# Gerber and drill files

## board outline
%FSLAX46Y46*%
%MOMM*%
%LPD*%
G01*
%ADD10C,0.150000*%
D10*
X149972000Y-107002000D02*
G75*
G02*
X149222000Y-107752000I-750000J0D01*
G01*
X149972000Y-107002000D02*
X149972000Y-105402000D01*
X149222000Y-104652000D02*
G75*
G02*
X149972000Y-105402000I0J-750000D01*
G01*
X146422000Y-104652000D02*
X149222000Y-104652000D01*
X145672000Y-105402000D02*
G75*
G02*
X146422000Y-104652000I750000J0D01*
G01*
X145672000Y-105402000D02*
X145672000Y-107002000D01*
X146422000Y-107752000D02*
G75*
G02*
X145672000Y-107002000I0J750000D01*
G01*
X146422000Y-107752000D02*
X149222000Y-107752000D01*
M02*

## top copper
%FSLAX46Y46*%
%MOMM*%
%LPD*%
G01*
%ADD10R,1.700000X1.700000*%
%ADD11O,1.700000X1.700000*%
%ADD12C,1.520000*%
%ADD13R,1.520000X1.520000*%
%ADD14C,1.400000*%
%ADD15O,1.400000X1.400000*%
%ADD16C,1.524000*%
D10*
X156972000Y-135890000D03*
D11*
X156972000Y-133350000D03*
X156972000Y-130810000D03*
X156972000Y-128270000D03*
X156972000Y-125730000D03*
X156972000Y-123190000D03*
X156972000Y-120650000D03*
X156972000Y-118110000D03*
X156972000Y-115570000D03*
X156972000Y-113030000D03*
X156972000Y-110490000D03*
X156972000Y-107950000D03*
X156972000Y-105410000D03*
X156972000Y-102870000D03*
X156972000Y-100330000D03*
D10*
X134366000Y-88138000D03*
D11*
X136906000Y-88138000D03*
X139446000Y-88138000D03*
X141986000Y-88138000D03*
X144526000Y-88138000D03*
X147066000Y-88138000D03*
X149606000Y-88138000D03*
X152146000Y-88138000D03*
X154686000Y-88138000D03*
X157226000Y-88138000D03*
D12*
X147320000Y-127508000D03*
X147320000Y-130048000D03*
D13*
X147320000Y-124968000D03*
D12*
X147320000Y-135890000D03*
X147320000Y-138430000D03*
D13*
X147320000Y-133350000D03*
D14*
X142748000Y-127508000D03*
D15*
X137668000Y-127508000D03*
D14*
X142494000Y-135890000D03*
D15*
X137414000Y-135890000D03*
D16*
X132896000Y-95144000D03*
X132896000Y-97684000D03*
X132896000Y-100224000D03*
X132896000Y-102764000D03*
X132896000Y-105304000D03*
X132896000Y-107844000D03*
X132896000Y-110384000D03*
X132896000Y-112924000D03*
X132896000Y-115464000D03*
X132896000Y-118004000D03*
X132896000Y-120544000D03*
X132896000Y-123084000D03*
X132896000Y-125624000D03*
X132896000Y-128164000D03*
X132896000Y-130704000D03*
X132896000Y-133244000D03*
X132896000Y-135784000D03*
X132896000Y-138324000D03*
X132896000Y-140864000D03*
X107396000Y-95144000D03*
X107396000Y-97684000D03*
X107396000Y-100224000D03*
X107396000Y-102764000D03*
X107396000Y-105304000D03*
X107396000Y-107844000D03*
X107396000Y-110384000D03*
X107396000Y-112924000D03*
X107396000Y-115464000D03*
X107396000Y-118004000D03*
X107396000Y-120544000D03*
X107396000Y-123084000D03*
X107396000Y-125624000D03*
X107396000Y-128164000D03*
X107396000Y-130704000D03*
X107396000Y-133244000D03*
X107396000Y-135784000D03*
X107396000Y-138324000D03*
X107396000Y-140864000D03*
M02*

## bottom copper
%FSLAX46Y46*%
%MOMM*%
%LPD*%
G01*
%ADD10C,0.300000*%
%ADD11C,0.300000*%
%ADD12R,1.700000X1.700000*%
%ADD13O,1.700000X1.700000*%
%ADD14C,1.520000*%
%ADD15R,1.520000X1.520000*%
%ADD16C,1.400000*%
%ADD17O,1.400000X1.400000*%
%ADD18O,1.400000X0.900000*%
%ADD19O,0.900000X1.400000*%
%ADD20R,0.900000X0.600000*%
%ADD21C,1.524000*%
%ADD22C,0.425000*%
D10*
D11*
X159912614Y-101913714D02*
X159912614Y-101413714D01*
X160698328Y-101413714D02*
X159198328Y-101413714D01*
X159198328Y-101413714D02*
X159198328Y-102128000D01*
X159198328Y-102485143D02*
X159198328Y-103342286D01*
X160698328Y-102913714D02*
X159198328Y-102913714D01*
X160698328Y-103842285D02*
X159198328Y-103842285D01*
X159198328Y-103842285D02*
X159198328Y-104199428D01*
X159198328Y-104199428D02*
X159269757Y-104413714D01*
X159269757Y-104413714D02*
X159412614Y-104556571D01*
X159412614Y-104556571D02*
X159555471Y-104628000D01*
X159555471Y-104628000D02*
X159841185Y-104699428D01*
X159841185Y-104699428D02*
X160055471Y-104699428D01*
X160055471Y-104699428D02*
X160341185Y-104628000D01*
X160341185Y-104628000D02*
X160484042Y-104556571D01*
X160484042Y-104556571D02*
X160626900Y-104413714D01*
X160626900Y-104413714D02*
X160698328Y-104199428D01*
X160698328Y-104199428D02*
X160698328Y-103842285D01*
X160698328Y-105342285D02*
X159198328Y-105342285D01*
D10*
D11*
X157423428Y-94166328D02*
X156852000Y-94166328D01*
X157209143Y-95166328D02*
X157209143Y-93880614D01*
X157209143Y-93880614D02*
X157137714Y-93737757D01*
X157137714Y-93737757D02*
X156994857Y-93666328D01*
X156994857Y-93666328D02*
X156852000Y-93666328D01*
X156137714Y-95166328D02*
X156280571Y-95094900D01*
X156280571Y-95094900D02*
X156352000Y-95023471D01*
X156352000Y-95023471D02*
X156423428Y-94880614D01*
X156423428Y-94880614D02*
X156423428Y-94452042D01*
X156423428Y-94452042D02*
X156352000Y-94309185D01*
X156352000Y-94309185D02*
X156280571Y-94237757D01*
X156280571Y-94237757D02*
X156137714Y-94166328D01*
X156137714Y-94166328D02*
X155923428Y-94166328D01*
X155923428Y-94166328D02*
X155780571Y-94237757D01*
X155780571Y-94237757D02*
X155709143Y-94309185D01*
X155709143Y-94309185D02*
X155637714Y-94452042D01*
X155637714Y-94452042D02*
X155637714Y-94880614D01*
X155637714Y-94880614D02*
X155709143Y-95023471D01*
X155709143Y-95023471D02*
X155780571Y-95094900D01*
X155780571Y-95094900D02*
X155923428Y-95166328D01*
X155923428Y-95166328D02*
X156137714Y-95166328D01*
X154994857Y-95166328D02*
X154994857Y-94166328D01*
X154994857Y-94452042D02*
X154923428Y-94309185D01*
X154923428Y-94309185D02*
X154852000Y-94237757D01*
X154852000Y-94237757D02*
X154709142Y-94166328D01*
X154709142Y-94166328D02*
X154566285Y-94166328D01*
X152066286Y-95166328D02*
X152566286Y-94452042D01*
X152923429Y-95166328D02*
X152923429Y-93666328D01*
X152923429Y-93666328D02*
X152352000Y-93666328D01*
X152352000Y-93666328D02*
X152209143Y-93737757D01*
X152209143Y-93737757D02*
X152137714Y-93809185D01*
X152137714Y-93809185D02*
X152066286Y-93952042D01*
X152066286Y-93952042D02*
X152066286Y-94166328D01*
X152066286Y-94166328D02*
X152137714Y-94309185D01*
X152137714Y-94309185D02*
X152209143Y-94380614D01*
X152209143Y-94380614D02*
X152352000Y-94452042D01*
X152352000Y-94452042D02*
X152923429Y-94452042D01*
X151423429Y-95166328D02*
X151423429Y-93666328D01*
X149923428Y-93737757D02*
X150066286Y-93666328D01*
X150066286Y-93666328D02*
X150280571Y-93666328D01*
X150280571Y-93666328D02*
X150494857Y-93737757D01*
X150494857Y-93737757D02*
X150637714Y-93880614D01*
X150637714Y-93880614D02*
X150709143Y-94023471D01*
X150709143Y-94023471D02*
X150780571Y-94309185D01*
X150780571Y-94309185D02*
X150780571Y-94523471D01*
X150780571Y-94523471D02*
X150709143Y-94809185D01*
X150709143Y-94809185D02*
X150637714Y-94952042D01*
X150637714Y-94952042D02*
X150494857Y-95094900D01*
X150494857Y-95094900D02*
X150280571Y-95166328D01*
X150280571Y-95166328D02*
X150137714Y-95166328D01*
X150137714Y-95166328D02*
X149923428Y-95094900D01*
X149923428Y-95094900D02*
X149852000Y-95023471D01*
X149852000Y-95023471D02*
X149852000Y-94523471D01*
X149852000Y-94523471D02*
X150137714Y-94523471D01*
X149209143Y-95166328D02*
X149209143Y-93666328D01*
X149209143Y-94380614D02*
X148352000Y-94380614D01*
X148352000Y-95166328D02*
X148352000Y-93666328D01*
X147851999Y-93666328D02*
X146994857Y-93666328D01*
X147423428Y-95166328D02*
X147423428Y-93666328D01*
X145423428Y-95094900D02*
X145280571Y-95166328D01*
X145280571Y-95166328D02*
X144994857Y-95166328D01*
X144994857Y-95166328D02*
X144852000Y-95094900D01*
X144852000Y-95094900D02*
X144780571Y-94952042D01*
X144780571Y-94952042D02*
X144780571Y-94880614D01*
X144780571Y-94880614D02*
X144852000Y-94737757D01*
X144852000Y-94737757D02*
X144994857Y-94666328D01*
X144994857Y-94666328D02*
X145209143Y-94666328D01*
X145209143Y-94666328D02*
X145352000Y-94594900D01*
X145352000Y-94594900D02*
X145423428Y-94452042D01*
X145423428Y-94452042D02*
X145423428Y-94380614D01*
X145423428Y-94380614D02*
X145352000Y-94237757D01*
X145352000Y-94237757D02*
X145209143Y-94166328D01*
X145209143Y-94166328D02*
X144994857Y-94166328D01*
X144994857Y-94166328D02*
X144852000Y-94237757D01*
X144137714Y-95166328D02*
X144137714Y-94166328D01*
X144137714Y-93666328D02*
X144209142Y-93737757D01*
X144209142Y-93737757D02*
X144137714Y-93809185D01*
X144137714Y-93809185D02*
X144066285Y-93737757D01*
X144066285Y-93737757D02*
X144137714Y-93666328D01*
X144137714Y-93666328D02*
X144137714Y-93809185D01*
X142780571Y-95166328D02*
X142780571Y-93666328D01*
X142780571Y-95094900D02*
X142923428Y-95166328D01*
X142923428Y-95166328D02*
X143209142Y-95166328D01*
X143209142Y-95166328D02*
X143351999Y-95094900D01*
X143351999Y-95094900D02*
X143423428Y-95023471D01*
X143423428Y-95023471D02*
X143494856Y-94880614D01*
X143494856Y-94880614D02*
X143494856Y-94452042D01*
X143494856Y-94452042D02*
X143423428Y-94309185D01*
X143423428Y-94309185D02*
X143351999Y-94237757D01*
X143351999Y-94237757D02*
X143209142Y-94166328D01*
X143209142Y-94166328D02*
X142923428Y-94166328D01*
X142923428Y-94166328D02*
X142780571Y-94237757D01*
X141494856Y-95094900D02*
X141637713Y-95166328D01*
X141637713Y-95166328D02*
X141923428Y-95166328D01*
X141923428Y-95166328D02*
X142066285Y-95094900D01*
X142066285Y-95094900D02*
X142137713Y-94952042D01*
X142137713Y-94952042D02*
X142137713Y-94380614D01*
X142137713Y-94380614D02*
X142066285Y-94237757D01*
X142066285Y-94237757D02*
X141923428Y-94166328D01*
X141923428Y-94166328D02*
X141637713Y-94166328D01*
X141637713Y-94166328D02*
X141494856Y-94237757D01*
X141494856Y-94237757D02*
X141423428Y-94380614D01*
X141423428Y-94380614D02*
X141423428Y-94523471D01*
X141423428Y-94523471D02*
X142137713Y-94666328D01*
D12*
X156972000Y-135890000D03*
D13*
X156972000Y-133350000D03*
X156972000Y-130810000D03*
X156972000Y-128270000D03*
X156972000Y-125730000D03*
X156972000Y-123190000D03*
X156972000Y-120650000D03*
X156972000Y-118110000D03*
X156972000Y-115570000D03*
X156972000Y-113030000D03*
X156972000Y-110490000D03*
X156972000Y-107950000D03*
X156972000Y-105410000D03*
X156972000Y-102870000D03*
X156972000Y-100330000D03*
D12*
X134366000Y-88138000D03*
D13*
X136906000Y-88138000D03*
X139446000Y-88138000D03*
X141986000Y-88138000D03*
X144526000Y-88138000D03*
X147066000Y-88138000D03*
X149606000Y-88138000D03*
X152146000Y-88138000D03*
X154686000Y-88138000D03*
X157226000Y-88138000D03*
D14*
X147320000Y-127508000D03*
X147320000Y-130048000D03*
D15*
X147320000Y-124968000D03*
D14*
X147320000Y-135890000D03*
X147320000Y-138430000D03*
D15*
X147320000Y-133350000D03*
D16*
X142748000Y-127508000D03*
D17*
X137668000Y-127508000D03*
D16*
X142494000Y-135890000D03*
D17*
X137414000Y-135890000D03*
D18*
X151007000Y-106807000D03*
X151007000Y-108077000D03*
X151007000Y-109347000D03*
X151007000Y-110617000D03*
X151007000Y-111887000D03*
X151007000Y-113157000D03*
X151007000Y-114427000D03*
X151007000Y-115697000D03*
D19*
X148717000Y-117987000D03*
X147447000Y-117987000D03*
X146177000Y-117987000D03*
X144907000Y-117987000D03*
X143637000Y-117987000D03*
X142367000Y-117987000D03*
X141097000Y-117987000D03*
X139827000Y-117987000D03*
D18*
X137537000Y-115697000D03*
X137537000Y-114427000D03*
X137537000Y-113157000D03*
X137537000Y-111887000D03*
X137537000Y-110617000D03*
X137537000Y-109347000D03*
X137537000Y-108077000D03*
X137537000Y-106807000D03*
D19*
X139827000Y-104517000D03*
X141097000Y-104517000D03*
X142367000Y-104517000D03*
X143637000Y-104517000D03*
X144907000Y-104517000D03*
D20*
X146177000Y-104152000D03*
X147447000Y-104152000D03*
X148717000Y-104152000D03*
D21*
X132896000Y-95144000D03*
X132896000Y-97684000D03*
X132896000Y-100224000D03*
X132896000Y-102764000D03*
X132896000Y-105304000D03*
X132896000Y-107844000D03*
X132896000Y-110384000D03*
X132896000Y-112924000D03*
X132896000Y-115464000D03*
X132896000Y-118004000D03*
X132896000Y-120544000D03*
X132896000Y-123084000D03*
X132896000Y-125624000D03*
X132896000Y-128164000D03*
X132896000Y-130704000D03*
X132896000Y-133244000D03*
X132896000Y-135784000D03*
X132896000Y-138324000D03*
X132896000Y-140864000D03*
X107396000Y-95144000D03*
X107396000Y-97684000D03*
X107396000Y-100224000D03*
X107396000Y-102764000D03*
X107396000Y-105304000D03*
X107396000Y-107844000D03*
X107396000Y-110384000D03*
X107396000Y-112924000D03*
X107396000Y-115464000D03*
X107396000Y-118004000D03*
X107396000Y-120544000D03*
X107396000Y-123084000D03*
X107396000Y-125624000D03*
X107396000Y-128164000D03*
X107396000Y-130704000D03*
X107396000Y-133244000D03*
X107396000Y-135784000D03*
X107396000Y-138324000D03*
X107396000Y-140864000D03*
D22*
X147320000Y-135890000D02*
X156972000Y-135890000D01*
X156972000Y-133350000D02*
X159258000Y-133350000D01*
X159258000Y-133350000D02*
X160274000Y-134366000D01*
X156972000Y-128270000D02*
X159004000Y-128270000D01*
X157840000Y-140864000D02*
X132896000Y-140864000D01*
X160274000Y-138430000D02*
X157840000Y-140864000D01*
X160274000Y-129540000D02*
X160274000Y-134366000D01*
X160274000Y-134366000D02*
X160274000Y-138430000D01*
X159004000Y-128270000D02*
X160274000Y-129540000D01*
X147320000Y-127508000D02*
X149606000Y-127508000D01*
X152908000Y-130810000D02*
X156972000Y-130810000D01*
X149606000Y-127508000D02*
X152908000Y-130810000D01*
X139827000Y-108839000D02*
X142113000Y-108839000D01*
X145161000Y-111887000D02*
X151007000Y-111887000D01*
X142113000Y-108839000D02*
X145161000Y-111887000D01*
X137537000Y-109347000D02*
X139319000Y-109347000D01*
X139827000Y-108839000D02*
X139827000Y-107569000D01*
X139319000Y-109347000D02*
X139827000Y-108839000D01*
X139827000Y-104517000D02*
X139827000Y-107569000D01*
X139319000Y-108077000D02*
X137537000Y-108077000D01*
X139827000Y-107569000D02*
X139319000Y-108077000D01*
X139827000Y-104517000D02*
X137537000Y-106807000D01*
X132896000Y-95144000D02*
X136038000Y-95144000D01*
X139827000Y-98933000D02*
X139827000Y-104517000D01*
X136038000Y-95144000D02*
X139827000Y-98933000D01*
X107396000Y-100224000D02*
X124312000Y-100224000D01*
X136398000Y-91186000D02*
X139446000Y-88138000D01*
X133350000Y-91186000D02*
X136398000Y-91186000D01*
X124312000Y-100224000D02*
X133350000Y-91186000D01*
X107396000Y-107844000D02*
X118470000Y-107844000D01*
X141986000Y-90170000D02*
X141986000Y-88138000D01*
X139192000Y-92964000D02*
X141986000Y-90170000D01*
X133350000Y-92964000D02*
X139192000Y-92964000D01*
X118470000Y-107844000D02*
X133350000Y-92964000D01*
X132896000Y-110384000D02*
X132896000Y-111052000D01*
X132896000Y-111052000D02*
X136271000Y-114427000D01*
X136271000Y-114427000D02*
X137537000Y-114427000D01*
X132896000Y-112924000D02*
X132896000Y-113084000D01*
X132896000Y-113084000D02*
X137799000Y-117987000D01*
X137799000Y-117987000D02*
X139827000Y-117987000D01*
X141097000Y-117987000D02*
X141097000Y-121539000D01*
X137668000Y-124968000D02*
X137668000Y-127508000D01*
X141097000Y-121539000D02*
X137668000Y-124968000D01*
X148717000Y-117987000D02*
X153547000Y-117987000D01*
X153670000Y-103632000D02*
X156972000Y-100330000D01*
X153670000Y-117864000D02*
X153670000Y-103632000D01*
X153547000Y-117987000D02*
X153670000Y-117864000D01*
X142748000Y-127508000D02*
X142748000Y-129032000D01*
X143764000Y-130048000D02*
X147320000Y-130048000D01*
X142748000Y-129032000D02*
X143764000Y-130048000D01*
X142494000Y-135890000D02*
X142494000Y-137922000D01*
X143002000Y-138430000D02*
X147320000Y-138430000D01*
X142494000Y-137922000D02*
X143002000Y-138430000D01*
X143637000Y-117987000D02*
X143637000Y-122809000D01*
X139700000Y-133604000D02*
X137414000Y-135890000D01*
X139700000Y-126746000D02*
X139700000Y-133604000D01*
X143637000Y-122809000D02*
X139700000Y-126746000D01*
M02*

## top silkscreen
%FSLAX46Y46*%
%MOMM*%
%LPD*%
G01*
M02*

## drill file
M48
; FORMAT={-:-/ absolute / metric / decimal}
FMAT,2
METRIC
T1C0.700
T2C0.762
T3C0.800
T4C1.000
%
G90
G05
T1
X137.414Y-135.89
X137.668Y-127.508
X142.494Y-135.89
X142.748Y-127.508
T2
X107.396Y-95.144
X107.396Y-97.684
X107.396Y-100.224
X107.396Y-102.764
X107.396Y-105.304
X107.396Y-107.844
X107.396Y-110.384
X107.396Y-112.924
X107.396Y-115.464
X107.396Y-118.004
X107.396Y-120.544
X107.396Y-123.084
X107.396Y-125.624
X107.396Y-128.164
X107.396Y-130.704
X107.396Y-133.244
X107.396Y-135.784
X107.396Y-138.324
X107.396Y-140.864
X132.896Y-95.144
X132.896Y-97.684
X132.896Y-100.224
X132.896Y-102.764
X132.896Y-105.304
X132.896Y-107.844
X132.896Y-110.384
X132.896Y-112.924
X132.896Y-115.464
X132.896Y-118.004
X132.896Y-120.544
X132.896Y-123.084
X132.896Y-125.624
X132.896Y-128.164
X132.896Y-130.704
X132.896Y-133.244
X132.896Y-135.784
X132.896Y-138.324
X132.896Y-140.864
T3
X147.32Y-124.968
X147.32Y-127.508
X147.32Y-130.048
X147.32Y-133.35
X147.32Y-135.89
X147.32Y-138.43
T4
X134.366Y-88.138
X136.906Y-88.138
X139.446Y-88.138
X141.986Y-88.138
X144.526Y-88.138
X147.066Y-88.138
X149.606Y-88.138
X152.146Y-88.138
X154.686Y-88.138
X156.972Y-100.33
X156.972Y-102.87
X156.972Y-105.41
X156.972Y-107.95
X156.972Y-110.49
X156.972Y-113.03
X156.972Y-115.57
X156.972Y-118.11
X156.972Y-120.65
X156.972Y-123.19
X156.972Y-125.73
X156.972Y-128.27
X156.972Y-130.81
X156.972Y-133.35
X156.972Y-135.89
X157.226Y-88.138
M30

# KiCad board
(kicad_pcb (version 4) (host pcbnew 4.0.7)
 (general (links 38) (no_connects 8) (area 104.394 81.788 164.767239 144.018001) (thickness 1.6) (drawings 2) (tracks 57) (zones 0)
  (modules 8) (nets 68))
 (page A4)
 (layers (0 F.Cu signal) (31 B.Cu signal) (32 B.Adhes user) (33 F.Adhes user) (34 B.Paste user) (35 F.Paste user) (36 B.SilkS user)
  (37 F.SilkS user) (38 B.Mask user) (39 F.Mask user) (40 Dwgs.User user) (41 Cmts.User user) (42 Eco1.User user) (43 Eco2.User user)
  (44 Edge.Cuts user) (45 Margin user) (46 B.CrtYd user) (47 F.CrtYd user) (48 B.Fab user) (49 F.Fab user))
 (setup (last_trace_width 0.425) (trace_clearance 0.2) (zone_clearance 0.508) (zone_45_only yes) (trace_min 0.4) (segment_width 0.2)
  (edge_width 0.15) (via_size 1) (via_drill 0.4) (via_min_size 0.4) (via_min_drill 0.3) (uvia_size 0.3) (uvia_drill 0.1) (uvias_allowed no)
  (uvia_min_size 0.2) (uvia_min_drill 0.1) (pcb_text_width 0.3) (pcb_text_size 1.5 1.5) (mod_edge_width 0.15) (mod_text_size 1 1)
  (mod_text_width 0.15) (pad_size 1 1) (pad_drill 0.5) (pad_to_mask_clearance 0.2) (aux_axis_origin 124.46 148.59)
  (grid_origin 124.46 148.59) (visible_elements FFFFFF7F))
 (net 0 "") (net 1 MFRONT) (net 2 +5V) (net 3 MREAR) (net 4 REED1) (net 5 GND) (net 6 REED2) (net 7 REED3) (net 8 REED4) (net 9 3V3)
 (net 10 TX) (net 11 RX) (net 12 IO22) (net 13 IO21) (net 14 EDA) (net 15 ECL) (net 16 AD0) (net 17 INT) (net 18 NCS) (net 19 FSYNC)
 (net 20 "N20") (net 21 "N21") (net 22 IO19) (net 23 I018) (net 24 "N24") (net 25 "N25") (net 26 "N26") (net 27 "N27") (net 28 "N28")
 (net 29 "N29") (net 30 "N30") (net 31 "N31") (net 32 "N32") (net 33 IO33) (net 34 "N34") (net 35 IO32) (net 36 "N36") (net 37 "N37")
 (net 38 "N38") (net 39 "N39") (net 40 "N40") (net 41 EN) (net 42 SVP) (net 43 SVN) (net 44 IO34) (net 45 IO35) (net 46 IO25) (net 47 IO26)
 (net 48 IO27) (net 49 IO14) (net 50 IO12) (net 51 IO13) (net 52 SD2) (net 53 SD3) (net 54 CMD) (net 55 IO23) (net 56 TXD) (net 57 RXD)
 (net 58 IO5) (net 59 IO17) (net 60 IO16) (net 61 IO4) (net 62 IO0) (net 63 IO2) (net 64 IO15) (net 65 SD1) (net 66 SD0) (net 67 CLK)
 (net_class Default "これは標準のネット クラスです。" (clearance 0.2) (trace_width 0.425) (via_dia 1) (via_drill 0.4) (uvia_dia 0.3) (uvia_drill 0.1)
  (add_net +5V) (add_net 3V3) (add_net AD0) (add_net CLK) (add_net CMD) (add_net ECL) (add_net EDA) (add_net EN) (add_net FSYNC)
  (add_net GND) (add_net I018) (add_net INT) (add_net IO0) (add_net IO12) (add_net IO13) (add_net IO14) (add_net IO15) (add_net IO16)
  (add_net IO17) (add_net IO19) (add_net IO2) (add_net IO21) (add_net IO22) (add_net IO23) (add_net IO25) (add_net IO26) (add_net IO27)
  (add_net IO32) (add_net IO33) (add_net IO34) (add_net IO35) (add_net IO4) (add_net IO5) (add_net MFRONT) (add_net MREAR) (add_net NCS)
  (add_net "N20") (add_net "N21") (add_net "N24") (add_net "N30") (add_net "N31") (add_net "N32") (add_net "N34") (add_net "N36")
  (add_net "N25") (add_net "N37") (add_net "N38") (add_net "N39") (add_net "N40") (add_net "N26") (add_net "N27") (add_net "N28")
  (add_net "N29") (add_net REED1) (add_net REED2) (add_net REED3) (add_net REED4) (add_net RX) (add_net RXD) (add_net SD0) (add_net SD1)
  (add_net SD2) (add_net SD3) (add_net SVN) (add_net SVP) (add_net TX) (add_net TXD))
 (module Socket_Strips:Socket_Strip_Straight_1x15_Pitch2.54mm (layer B.Cu) (at 156.972 135.89)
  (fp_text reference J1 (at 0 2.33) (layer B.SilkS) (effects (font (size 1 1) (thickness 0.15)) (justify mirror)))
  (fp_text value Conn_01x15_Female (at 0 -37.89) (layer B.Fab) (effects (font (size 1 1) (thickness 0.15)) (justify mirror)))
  (pad 1 thru_hole rect (at 0 0) (size 1.7 1.7) (drill 1) (layers *.Cu *.Mask) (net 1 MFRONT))
  (pad 2 thru_hole oval (at 0 -2.54) (size 1.7 1.7) (drill 1) (layers *.Cu *.Mask) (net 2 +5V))
  (pad 3 thru_hole oval (at 0 -5.08) (size 1.7 1.7) (drill 1) (layers *.Cu *.Mask) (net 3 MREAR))
  (pad 4 thru_hole oval (at 0 -7.62) (size 1.7 1.7) (drill 1) (layers *.Cu *.Mask) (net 2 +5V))
  (pad 5 thru_hole oval (at 0 -10.16) (size 1.7 1.7) (drill 1) (layers *.Cu *.Mask) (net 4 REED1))
  (pad 6 thru_hole oval (at 0 -12.7) (size 1.7 1.7) (drill 1) (layers *.Cu *.Mask) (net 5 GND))
  (pad 7 thru_hole oval (at 0 -15.24) (size 1.7 1.7) (drill 1) (layers *.Cu *.Mask) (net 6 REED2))
  (pad 8 thru_hole oval (at 0 -17.78) (size 1.7 1.7) (drill 1) (layers *.Cu *.Mask) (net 5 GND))
  (pad 9 thru_hole oval (at 0 -20.32) (size 1.7 1.7) (drill 1) (layers *.Cu *.Mask) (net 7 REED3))
  (pad 10 thru_hole oval (at 0 -22.86) (size 1.7 1.7) (drill 1) (layers *.Cu *.Mask) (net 5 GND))
  (pad 11 thru_hole oval (at 0 -25.4) (size 1.7 1.7) (drill 1) (layers *.Cu *.Mask) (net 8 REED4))
  (pad 12 thru_hole oval (at 0 -27.94) (size 1.7 1.7) (drill 1) (layers *.Cu *.Mask) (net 5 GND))
  (pad 13 thru_hole oval (at 0 -30.48) (size 1.7 1.7) (drill 1) (layers *.Cu *.Mask) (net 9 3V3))
  (pad 14 thru_hole oval (at 0 -33.02) (size 1.7 1.7) (drill 1) (layers *.Cu *.Mask) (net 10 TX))
  (pad 15 thru_hole oval (at 0 -35.56) (size 1.7 1.7) (drill 1) (layers *.Cu *.Mask) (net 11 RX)))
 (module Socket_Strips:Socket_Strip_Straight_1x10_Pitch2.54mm (layer B.Cu) (at 134.366 88.138 270)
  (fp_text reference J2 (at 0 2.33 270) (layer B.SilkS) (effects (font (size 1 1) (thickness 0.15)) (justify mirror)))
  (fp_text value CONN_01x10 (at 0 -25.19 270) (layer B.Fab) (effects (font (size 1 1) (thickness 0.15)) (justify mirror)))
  (pad 1 thru_hole rect (at 0 0 270) (size 1.7 1.7) (drill 1) (layers *.Cu *.Mask) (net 9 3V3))
  (pad 2 thru_hole oval (at 0 -2.54 270) (size 1.7 1.7) (drill 1) (layers *.Cu *.Mask) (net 5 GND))
  (pad 3 thru_hole oval (at 0 -5.08 270) (size 1.7 1.7) (drill 1) (layers *.Cu *.Mask) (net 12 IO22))
  (pad 4 thru_hole oval (at 0 -7.62 270) (size 1.7 1.7) (drill 1) (layers *.Cu *.Mask) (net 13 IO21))
  (pad 5 thru_hole oval (at 0 -10.16 270) (size 1.7 1.7) (drill 1) (layers *.Cu *.Mask) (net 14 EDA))
  (pad 6 thru_hole oval (at 0 -12.7 270) (size 1.7 1.7) (drill 1) (layers *.Cu *.Mask) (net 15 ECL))
  (pad 7 thru_hole oval (at 0 -15.24 270) (size 1.7 1.7) (drill 1) (layers *.Cu *.Mask) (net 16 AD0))
  (pad 8 thru_hole oval (at 0 -17.78 270) (size 1.7 1.7) (drill 1) (layers *.Cu *.Mask) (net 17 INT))
  (pad 9 thru_hole oval (at 0 -20.32 270) (size 1.7 1.7) (drill 1) (layers *.Cu *.Mask) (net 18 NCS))
  (pad 10 thru_hole oval (at 0 -22.86 270) (size 1.7 1.7) (drill 1) (layers *.Cu *.Mask) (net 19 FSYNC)))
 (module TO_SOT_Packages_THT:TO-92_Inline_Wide (layer B.Cu) (at 147.32 124.968 270)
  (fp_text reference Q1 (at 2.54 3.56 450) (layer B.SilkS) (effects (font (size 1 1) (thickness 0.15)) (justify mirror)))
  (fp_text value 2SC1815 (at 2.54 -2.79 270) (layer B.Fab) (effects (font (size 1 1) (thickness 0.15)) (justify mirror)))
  (pad 2 thru_hole circle (at 2.54 0 180) (size 1.52 1.52) (drill 0.8) (layers *.Cu *.Mask) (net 3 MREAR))
  (pad 3 thru_hole circle (at 5.08 0 180) (size 1.52 1.52) (drill 0.8) (layers *.Cu *.Mask) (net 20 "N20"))
  (pad 1 thru_hole rect (at 0 0 180) (size 1.52 1.52) (drill 0.8) (layers *.Cu *.Mask) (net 5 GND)))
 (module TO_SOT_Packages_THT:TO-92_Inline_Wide (layer B.Cu) (at 147.32 133.35 270)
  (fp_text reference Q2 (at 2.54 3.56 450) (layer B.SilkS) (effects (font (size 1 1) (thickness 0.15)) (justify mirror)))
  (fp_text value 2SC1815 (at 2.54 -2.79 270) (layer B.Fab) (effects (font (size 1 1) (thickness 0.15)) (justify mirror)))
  (pad 2 thru_hole circle (at 2.54 0 180) (size 1.52 1.52) (drill 0.8) (layers *.Cu *.Mask) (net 1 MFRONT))
  (pad 3 thru_hole circle (at 5.08 0 180) (size 1.52 1.52) (drill 0.8) (layers *.Cu *.Mask) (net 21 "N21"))
  (pad 1 thru_hole rect (at 0 0 180) (size 1.52 1.52) (drill 0.8) (layers *.Cu *.Mask) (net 5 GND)))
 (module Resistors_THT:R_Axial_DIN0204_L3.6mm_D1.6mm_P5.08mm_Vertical (layer B.Cu) (at 142.748 127.508 180)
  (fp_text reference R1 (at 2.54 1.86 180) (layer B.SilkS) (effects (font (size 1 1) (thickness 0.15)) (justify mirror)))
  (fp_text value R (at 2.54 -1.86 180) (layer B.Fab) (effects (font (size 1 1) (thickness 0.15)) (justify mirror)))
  (pad 1 thru_hole circle (at 0 0 180) (size 1.4 1.4) (drill 0.7) (layers *.Cu *.Mask) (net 20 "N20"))
  (pad 2 thru_hole oval (at 5.08 0 180) (size 1.4 1.4) (drill 0.7) (layers *.Cu *.Mask) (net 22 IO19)))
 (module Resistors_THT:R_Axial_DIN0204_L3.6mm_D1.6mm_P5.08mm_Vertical (layer B.Cu) (at 142.494 135.89 180)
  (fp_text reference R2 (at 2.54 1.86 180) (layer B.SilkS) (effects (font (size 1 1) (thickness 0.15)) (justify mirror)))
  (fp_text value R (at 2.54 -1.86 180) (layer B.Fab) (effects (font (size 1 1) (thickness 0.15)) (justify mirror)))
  (pad 1 thru_hole circle (at 0 0 180) (size 1.4 1.4) (drill 0.7) (layers *.Cu *.Mask) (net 21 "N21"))
  (pad 2 thru_hole oval (at 5.08 0 180) (size 1.4 1.4) (drill 0.7) (layers *.Cu *.Mask) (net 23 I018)))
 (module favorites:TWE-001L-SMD (layer B.Cu) (at 144.272 111.252 180)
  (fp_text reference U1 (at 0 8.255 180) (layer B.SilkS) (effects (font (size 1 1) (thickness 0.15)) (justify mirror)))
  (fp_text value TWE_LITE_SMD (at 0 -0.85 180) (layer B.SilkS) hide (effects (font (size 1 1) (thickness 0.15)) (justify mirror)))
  (fp_arc (start -4.95 4.25) (end -4.95 3.5) (angle -90) (layer Edge.Cuts) (width 0.15))
  (fp_line (start -5.7 4.25) (end -5.7 5.85) (layer Edge.Cuts) (width 0.15))
  (fp_arc (start -4.95 5.85) (end -5.7 5.85) (angle -90) (layer Edge.Cuts) (width 0.15))
  (fp_line (start -2.15 6.6) (end -4.95 6.6) (layer Edge.Cuts) (width 0.15))
  (fp_arc (start -2.15 5.85) (end -2.15 6.6) (angle -90) (layer Edge.Cuts) (width 0.15))
  (fp_line (start -1.4 5.85) (end -1.4 4.25) (layer Edge.Cuts) (width 0.15))
  (fp_arc (start -2.15 4.25) (end -1.4 4.25) (angle -90) (layer Edge.Cuts) (width 0.15))
  (fp_line (start -2.15 3.5) (end -4.95 3.5) (layer Edge.Cuts) (width 0.15))
  (pad 1 smd oval (at -6.735 4.445 90) (size 0.9 1.4) (layers B.Cu B.Paste B.Mask) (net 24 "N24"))
  (pad 2 smd oval (at -6.735 3.175 90) (size 0.9 1.4) (layers B.Cu B.Paste B.Mask) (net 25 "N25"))
  (pad 3 smd oval (at -6.735 1.905 90) (size 0.9 1.4) (layers B.Cu B.Paste B.Mask) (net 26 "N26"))
  (pad 4 smd oval (at -6.735 0.635 90) (size 0.9 1.4) (layers B.Cu B.Paste B.Mask) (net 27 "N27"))
  (pad 5 smd oval (at -6.735 -0.635 90) (size 0.9 1.4) (layers B.Cu B.Paste B.Mask) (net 9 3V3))
  (pad 6 smd oval (at -6.735 -1.905 90) (size 0.9 1.4) (layers B.Cu B.Paste B.Mask) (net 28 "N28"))
  (pad 7 smd oval (at -6.735 -3.175 90) (size 0.9 1.4) (layers B.Cu B.Paste B.Mask) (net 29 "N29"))
  (pad 8 smd oval (at -6.735 -4.445 90) (size 0.9 1.4) (layers B.Cu B.Paste B.Mask) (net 10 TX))
  (pad 9 smd oval (at -4.445 -6.735 180) (size 0.9 1.4) (layers B.Cu B.Paste B.Mask) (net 11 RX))
  (pad 10 smd oval (at -3.175 -6.735 180) (size 0.9 1.4) (layers B.Cu B.Paste B.Mask) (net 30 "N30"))
  (pad 11 smd oval (at -1.905 -6.735 180) (size 0.9 1.4) (layers B.Cu B.Paste B.Mask) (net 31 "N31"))
  (pad 12 smd oval (at -0.635 -6.735 180) (size 0.9 1.4) (layers B.Cu B.Paste B.Mask) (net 5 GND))
  (pad 13 smd oval (at 0.635 -6.735 180) (size 0.9 1.4) (layers B.Cu B.Paste B.Mask) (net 23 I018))
  (pad 14 smd oval (at 1.905 -6.735 180) (size 0.9 1.4) (layers B.Cu B.Paste B.Mask) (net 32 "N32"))
  (pad 15 smd oval (at 3.175 -6.735 180) (size 0.9 1.4) (layers B.Cu B.Paste B.Mask) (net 22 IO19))
  (pad 16 smd oval (at 4.445 -6.735 180) (size 0.9 1.4) (layers B.Cu B.Paste B.Mask) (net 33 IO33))
  (pad 17 smd oval (at 6.735 -4.445 90) (size 0.9 1.4) (layers B.Cu B.Paste B.Mask) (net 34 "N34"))
  (pad 18 smd oval (at 6.735 -3.175 90) (size 0.9 1.4) (layers B.Cu B.Paste B.Mask) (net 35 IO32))
  (pad 19 smd oval (at 6.735 -1.905 90) (size 0.9 1.4) (layers B.Cu B.Paste B.Mask) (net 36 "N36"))
  (pad 20 smd oval (at 6.735 -0.635 90) (size 0.9 1.4) (layers B.Cu B.Paste B.Mask) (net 5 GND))
  (pad 21 smd oval (at 6.735 0.635 90) (size 0.9 1.4) (layers B.Cu B.Paste B.Mask) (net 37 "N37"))
  (pad 22 smd oval (at 6.735 1.905 90) (size 0.9 1.4) (layers B.Cu B.Paste B.Mask) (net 9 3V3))
  (pad 23 smd oval (at 6.735 3.175 90) (size 0.9 1.4) (layers B.Cu B.Paste B.Mask) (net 9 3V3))
  (pad 24 smd oval (at 6.735 4.445 90) (size 0.9 1.4) (layers B.Cu B.Paste B.Mask) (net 9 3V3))
  (pad 25 smd oval (at 4.445 6.735 180) (size 0.9 1.4) (layers B.Cu B.Paste B.Mask) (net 9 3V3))
  (pad 26 smd oval (at 3.175 6.735 180) (size 0.9 1.4) (layers B.Cu B.Paste B.Mask) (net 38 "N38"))
  (pad 27 smd oval (at 1.905 6.735 180) (size 0.9 1.4) (layers B.Cu B.Paste B.Mask) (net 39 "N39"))
  (pad 28 smd oval (at 0.635 6.735 180) (size 0.9 1.4) (layers B.Cu B.Paste B.Mask) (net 5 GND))
  (pad 29 smd oval (at -0.635 6.735 180) (size 0.9 1.4) (layers B.Cu B.Paste B.Mask) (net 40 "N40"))
  (pad 30 smd rect (at -1.905 7.1 180) (size 0.9 0.6) (layers B.Cu B.Paste B.Mask) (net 5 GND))
  (pad 31 smd rect (at -3.175 7.1 180) (size 0.9 0.6) (layers B.Cu B.Paste B.Mask) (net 5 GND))
  (pad 32 smd rect (at -4.445 7.1 180) (size 0.9 0.6) (layers B.Cu B.Paste B.Mask) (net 5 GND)))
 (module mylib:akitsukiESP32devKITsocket (layer B.Cu) (at 120.396 123.444 180)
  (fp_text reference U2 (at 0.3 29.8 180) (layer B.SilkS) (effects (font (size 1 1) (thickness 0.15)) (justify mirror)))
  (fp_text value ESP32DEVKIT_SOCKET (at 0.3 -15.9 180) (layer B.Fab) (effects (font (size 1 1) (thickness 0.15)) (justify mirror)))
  (pad 1 thru_hole circle (at -12.5 28.3 180) (size 1.524 1.524) (drill 0.762) (layers *.Cu *.Mask) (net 9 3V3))
  (pad 2 thru_hole circle (at -12.5 25.76 180) (size 1.524 1.524) (drill 0.762) (layers *.Cu *.Mask) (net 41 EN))
  (pad 3 thru_hole circle (at -12.5 23.22 180) (size 1.524 1.524) (drill 0.762) (layers *.Cu *.Mask) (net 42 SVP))
  (pad 4 thru_hole circle (at -12.5 20.68 180) (size 1.524 1.524) (drill 0.762) (layers *.Cu *.Mask) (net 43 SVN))
  (pad 5 thru_hole circle (at -12.5 18.14 180) (size 1.524 1.524) (drill 0.762) (layers *.Cu *.Mask) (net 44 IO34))
  (pad 6 thru_hole circle (at -12.5 15.6 180) (size 1.524 1.524) (drill 0.762) (layers *.Cu *.Mask) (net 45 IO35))
  (pad 7 thru_hole circle (at -12.5 13.06 180) (size 1.524 1.524) (drill 0.762) (layers *.Cu *.Mask) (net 35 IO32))
  (pad 8 thru_hole circle (at -12.5 10.52 180) (size 1.524 1.524) (drill 0.762) (layers *.Cu *.Mask) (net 33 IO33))
  (pad 9 thru_hole circle (at -12.5 7.98 180) (size 1.524 1.524) (drill 0.762) (layers *.Cu *.Mask) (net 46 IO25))
  (pad 10 thru_hole circle (at -12.5 5.44 180) (size 1.524 1.524) (drill 0.762) (layers *.Cu *.Mask) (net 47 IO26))
  (pad 11 thru_hole circle (at -12.5 2.9 180) (size 1.524 1.524) (drill 0.762) (layers *.Cu *.Mask) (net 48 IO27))
  (pad 12 thru_hole circle (at -12.5 0.36 180) (size 1.524 1.524) (drill 0.762) (layers *.Cu *.Mask) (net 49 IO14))
  (pad 13 thru_hole circle (at -12.5 -2.18 180) (size 1.524 1.524) (drill 0.762) (layers *.Cu *.Mask) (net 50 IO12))
  (pad 14 thru_hole circle (at -12.5 -4.72 180) (size 1.524 1.524) (drill 0.762) (layers *.Cu *.Mask) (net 5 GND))
  (pad 15 thru_hole circle (at -12.5 -7.26 180) (size 1.524 1.524) (drill 0.762) (layers *.Cu *.Mask) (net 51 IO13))
  (pad 16 thru_hole circle (at -12.5 -9.8 180) (size 1.524 1.524) (drill 0.762) (layers *.Cu *.Mask) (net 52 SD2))
  (pad 17 thru_hole circle (at -12.5 -12.34 180) (size 1.524 1.524) (drill 0.762) (layers *.Cu *.Mask) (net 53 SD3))
  (pad 18 thru_hole circle (at -12.5 -14.88 180) (size 1.524 1.524) (drill 0.762) (layers *.Cu *.Mask) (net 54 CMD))
  (pad 19 thru_hole circle (at -12.5 -17.42 180) (size 1.524 1.524) (drill 0.762) (layers *.Cu *.Mask) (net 2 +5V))
  (pad 20 thru_hole circle (at 13 28.3 180) (size 1.524 1.524) (drill 0.762) (layers *.Cu *.Mask) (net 5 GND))
  (pad 21 thru_hole circle (at 13 25.76 180) (size 1.524 1.524) (drill 0.762) (layers *.Cu *.Mask) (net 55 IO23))
  (pad 22 thru_hole circle (at 13 23.22 180) (size 1.524 1.524) (drill 0.762) (layers *.Cu *.Mask) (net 12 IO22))
  (pad 23 thru_hole circle (at 13 20.68 180) (size 1.524 1.524) (drill 0.762) (layers *.Cu *.Mask) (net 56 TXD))
  (pad 24 thru_hole circle (at 13 18.14 180) (size 1.524 1.524) (drill 0.762) (layers *.Cu *.Mask) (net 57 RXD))
  (pad 25 thru_hole circle (at 13 15.6 180) (size 1.524 1.524) (drill 0.762) (layers *.Cu *.Mask) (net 13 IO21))
  (pad 26 thru_hole circle (at 13 13.06 180) (size 1.524 1.524) (drill 0.762) (layers *.Cu *.Mask) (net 5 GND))
  (pad 27 thru_hole circle (at 13 10.52 180) (size 1.524 1.524) (drill 0.762) (layers *.Cu *.Mask) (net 22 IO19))
  (pad 28 thru_hole circle (at 13 7.98 180) (size 1.524 1.524) (drill 0.762) (layers *.Cu *.Mask) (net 23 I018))
  (pad 29 thru_hole circle (at 13 5.44 180) (size 1.524 1.524) (drill 0.762) (layers *.Cu *.Mask) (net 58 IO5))
  (pad 30 thru_hole circle (at 13 2.9 180) (size 1.524 1.524) (drill 0.762) (layers *.Cu *.Mask) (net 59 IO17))
  (pad 31 thru_hole circle (at 13 0.36 180) (size 1.524 1.524) (drill 0.762) (layers *.Cu *.Mask) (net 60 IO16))
  (pad 32 thru_hole circle (at 13 -2.18 180) (size 1.524 1.524) (drill 0.762) (layers *.Cu *.Mask) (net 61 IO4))
  (pad 33 thru_hole circle (at 13 -4.72 180) (size 1.524 1.524) (drill 0.762) (layers *.Cu *.Mask) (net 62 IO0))
  (pad 34 thru_hole circle (at 13 -7.26 180) (size 1.524 1.524) (drill 0.762) (layers *.Cu *.Mask) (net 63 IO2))
  (pad 35 thru_hole circle (at 13 -9.8 180) (size 1.524 1.524) (drill 0.762) (layers *.Cu *.Mask) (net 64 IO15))
  (pad 36 thru_hole circle (at 13 -12.34 180) (size 1.524 1.524) (drill 0.762) (layers *.Cu *.Mask) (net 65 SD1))
  (pad 37 thru_hole circle (at 13 -14.88 180) (size 1.524 1.524) (drill 0.762) (layers *.Cu *.Mask) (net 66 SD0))
  (pad 38 thru_hole circle (at 13 -17.42 180) (size 1.524 1.524) (drill 0.762) (layers *.Cu *.Mask) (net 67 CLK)))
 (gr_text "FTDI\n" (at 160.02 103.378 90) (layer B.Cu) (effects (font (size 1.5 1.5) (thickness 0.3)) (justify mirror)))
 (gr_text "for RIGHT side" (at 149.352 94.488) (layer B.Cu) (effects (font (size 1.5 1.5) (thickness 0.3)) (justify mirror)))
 (segment (start 147.32 135.89) (end 156.972 135.89) (width 0.425) (layer B.Cu) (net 1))
 (segment (start 156.972 133.35) (end 159.258 133.35) (width 0.425) (layer B.Cu) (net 2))
 (segment (start 159.258 133.35) (end 160.274 134.366) (width 0.425) (layer B.Cu) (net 2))
 (segment (start 156.972 128.27) (end 159.004 128.27) (width 0.425) (layer B.Cu) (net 2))
 (segment (start 157.84 140.864) (end 132.896 140.864) (width 0.425) (layer B.Cu) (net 2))
 (segment (start 160.274 138.43) (end 157.84 140.864) (width 0.425) (layer B.Cu) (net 2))
 (segment (start 160.274 129.54) (end 160.274 134.366) (width 0.425) (layer B.Cu) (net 2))
 (segment (start 160.274 134.366) (end 160.274 138.43) (width 0.425) (layer B.Cu) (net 2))
 (segment (start 159.004 128.27) (end 160.274 129.54) (width 0.425) (layer B.Cu) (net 2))
 (segment (start 147.32 127.508) (end 149.606 127.508) (width 0.425) (layer B.Cu) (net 3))
 (segment (start 152.908 130.81) (end 156.972 130.81) (width 0.425) (layer B.Cu) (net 3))
 (segment (start 149.606 127.508) (end 152.908 130.81) (width 0.425) (layer B.Cu) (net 3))
 (segment (start 139.827 108.839) (end 142.113 108.839) (width 0.425) (layer B.Cu) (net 9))
 (segment (start 145.161 111.887) (end 151.007 111.887) (width 0.425) (layer B.Cu) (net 9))
 (segment (start 142.113 108.839) (end 145.161 111.887) (width 0.425) (layer B.Cu) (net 9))
 (segment (start 137.537 109.347) (end 139.319 109.347) (width 0.425) (layer B.Cu) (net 9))
 (segment (start 139.827 108.839) (end 139.827 107.569) (width 0.425) (layer B.Cu) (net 9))
 (segment (start 139.319 109.347) (end 139.827 108.839) (width 0.425) (layer B.Cu) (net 9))
 (segment (start 139.827 104.517) (end 139.827 107.569) (width 0.425) (layer B.Cu) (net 9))
 (segment (start 139.319 108.077) (end 137.537 108.077) (width 0.425) (layer B.Cu) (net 9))
 (segment (start 139.827 107.569) (end 139.319 108.077) (width 0.425) (layer B.Cu) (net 9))
 (segment (start 139.827 104.517) (end 137.537 106.807) (width 0.425) (layer B.Cu) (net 9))
 (segment (start 132.896 95.144) (end 136.038 95.144) (width 0.425) (layer B.Cu) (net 9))
 (segment (start 139.827 98.933) (end 139.827 104.517) (width 0.425) (layer B.Cu) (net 9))
 (segment (start 136.038 95.144) (end 139.827 98.933) (width 0.425) (layer B.Cu) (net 9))
 (segment (start 107.396 100.224) (end 124.312 100.224) (width 0.425) (layer B.Cu) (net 12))
 (segment (start 136.398 91.186) (end 139.446 88.138) (width 0.425) (layer B.Cu) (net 12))
 (segment (start 133.35 91.186) (end 136.398 91.186) (width 0.425) (layer B.Cu) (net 12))
 (segment (start 124.312 100.224) (end 133.35 91.186) (width 0.425) (layer B.Cu) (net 12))
 (segment (start 107.396 107.844) (end 118.47 107.844) (width 0.425) (layer B.Cu) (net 13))
 (segment (start 141.986 90.17) (end 141.986 88.138) (width 0.425) (layer B.Cu) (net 13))
 (segment (start 139.192 92.964) (end 141.986 90.17) (width 0.425) (layer B.Cu) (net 13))
 (segment (start 133.35 92.964) (end 139.192 92.964) (width 0.425) (layer B.Cu) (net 13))
 (segment (start 118.47 107.844) (end 133.35 92.964) (width 0.425) (layer B.Cu) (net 13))
 (segment (start 132.896 110.384) (end 132.896 111.052) (width 0.425) (layer B.Cu) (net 35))
 (segment (start 132.896 111.052) (end 136.271 114.427) (width 0.425) (layer B.Cu) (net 35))
 (segment (start 136.271 114.427) (end 137.537 114.427) (width 0.425) (layer B.Cu) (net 35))
 (segment (start 132.896 112.924) (end 132.896 113.084) (width 0.425) (layer B.Cu) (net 33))
 (segment (start 132.896 113.084) (end 137.799 117.987) (width 0.425) (layer B.Cu) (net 33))
 (segment (start 137.799 117.987) (end 139.827 117.987) (width 0.425) (layer B.Cu) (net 33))
 (segment (start 141.097 117.987) (end 141.097 121.539) (width 0.425) (layer B.Cu) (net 22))
 (segment (start 137.668 124.968) (end 137.668 127.508) (width 0.425) (layer B.Cu) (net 22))
 (segment (start 141.097 121.539) (end 137.668 124.968) (width 0.425) (layer B.Cu) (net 22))
 (segment (start 148.717 117.987) (end 153.547 117.987) (width 0.425) (layer B.Cu) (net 11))
 (segment (start 153.67 103.632) (end 156.972 100.33) (width 0.425) (layer B.Cu) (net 11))
 (segment (start 153.67 117.864) (end 153.67 103.632) (width 0.425) (layer B.Cu) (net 11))
 (segment (start 153.547 117.987) (end 153.67 117.864) (width 0.425) (layer B.Cu) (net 11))
 (segment (start 142.748 127.508) (end 142.748 129.032) (width 0.425) (layer B.Cu) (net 20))
 (segment (start 143.764 130.048) (end 147.32 130.048) (width 0.425) (layer B.Cu) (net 20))
 (segment (start 142.748 129.032) (end 143.764 130.048) (width 0.425) (layer B.Cu) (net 20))
 (segment (start 142.494 135.89) (end 142.494 137.922) (width 0.425) (layer B.Cu) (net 21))
 (segment (start 143.002 138.43) (end 147.32 138.43) (width 0.425) (layer B.Cu) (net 21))
 (segment (start 142.494 137.922) (end 143.002 138.43) (width 0.425) (layer B.Cu) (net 21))
 (segment (start 143.637 117.987) (end 143.637 122.809) (width 0.425) (layer B.Cu) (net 23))
 (segment (start 139.7 133.604) (end 137.414 135.89) (width 0.425) (layer B.Cu) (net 23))
 (segment (start 139.7 126.746) (end 139.7 133.604) (width 0.425) (layer B.Cu) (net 23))
 (segment (start 143.637 122.809) (end 139.7 126.746) (width 0.425) (layer B.Cu) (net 23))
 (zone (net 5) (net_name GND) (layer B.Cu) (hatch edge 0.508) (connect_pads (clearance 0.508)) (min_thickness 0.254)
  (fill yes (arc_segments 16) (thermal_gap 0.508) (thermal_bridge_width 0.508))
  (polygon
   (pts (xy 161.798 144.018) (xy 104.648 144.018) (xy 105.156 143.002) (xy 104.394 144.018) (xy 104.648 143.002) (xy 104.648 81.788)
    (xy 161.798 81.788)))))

